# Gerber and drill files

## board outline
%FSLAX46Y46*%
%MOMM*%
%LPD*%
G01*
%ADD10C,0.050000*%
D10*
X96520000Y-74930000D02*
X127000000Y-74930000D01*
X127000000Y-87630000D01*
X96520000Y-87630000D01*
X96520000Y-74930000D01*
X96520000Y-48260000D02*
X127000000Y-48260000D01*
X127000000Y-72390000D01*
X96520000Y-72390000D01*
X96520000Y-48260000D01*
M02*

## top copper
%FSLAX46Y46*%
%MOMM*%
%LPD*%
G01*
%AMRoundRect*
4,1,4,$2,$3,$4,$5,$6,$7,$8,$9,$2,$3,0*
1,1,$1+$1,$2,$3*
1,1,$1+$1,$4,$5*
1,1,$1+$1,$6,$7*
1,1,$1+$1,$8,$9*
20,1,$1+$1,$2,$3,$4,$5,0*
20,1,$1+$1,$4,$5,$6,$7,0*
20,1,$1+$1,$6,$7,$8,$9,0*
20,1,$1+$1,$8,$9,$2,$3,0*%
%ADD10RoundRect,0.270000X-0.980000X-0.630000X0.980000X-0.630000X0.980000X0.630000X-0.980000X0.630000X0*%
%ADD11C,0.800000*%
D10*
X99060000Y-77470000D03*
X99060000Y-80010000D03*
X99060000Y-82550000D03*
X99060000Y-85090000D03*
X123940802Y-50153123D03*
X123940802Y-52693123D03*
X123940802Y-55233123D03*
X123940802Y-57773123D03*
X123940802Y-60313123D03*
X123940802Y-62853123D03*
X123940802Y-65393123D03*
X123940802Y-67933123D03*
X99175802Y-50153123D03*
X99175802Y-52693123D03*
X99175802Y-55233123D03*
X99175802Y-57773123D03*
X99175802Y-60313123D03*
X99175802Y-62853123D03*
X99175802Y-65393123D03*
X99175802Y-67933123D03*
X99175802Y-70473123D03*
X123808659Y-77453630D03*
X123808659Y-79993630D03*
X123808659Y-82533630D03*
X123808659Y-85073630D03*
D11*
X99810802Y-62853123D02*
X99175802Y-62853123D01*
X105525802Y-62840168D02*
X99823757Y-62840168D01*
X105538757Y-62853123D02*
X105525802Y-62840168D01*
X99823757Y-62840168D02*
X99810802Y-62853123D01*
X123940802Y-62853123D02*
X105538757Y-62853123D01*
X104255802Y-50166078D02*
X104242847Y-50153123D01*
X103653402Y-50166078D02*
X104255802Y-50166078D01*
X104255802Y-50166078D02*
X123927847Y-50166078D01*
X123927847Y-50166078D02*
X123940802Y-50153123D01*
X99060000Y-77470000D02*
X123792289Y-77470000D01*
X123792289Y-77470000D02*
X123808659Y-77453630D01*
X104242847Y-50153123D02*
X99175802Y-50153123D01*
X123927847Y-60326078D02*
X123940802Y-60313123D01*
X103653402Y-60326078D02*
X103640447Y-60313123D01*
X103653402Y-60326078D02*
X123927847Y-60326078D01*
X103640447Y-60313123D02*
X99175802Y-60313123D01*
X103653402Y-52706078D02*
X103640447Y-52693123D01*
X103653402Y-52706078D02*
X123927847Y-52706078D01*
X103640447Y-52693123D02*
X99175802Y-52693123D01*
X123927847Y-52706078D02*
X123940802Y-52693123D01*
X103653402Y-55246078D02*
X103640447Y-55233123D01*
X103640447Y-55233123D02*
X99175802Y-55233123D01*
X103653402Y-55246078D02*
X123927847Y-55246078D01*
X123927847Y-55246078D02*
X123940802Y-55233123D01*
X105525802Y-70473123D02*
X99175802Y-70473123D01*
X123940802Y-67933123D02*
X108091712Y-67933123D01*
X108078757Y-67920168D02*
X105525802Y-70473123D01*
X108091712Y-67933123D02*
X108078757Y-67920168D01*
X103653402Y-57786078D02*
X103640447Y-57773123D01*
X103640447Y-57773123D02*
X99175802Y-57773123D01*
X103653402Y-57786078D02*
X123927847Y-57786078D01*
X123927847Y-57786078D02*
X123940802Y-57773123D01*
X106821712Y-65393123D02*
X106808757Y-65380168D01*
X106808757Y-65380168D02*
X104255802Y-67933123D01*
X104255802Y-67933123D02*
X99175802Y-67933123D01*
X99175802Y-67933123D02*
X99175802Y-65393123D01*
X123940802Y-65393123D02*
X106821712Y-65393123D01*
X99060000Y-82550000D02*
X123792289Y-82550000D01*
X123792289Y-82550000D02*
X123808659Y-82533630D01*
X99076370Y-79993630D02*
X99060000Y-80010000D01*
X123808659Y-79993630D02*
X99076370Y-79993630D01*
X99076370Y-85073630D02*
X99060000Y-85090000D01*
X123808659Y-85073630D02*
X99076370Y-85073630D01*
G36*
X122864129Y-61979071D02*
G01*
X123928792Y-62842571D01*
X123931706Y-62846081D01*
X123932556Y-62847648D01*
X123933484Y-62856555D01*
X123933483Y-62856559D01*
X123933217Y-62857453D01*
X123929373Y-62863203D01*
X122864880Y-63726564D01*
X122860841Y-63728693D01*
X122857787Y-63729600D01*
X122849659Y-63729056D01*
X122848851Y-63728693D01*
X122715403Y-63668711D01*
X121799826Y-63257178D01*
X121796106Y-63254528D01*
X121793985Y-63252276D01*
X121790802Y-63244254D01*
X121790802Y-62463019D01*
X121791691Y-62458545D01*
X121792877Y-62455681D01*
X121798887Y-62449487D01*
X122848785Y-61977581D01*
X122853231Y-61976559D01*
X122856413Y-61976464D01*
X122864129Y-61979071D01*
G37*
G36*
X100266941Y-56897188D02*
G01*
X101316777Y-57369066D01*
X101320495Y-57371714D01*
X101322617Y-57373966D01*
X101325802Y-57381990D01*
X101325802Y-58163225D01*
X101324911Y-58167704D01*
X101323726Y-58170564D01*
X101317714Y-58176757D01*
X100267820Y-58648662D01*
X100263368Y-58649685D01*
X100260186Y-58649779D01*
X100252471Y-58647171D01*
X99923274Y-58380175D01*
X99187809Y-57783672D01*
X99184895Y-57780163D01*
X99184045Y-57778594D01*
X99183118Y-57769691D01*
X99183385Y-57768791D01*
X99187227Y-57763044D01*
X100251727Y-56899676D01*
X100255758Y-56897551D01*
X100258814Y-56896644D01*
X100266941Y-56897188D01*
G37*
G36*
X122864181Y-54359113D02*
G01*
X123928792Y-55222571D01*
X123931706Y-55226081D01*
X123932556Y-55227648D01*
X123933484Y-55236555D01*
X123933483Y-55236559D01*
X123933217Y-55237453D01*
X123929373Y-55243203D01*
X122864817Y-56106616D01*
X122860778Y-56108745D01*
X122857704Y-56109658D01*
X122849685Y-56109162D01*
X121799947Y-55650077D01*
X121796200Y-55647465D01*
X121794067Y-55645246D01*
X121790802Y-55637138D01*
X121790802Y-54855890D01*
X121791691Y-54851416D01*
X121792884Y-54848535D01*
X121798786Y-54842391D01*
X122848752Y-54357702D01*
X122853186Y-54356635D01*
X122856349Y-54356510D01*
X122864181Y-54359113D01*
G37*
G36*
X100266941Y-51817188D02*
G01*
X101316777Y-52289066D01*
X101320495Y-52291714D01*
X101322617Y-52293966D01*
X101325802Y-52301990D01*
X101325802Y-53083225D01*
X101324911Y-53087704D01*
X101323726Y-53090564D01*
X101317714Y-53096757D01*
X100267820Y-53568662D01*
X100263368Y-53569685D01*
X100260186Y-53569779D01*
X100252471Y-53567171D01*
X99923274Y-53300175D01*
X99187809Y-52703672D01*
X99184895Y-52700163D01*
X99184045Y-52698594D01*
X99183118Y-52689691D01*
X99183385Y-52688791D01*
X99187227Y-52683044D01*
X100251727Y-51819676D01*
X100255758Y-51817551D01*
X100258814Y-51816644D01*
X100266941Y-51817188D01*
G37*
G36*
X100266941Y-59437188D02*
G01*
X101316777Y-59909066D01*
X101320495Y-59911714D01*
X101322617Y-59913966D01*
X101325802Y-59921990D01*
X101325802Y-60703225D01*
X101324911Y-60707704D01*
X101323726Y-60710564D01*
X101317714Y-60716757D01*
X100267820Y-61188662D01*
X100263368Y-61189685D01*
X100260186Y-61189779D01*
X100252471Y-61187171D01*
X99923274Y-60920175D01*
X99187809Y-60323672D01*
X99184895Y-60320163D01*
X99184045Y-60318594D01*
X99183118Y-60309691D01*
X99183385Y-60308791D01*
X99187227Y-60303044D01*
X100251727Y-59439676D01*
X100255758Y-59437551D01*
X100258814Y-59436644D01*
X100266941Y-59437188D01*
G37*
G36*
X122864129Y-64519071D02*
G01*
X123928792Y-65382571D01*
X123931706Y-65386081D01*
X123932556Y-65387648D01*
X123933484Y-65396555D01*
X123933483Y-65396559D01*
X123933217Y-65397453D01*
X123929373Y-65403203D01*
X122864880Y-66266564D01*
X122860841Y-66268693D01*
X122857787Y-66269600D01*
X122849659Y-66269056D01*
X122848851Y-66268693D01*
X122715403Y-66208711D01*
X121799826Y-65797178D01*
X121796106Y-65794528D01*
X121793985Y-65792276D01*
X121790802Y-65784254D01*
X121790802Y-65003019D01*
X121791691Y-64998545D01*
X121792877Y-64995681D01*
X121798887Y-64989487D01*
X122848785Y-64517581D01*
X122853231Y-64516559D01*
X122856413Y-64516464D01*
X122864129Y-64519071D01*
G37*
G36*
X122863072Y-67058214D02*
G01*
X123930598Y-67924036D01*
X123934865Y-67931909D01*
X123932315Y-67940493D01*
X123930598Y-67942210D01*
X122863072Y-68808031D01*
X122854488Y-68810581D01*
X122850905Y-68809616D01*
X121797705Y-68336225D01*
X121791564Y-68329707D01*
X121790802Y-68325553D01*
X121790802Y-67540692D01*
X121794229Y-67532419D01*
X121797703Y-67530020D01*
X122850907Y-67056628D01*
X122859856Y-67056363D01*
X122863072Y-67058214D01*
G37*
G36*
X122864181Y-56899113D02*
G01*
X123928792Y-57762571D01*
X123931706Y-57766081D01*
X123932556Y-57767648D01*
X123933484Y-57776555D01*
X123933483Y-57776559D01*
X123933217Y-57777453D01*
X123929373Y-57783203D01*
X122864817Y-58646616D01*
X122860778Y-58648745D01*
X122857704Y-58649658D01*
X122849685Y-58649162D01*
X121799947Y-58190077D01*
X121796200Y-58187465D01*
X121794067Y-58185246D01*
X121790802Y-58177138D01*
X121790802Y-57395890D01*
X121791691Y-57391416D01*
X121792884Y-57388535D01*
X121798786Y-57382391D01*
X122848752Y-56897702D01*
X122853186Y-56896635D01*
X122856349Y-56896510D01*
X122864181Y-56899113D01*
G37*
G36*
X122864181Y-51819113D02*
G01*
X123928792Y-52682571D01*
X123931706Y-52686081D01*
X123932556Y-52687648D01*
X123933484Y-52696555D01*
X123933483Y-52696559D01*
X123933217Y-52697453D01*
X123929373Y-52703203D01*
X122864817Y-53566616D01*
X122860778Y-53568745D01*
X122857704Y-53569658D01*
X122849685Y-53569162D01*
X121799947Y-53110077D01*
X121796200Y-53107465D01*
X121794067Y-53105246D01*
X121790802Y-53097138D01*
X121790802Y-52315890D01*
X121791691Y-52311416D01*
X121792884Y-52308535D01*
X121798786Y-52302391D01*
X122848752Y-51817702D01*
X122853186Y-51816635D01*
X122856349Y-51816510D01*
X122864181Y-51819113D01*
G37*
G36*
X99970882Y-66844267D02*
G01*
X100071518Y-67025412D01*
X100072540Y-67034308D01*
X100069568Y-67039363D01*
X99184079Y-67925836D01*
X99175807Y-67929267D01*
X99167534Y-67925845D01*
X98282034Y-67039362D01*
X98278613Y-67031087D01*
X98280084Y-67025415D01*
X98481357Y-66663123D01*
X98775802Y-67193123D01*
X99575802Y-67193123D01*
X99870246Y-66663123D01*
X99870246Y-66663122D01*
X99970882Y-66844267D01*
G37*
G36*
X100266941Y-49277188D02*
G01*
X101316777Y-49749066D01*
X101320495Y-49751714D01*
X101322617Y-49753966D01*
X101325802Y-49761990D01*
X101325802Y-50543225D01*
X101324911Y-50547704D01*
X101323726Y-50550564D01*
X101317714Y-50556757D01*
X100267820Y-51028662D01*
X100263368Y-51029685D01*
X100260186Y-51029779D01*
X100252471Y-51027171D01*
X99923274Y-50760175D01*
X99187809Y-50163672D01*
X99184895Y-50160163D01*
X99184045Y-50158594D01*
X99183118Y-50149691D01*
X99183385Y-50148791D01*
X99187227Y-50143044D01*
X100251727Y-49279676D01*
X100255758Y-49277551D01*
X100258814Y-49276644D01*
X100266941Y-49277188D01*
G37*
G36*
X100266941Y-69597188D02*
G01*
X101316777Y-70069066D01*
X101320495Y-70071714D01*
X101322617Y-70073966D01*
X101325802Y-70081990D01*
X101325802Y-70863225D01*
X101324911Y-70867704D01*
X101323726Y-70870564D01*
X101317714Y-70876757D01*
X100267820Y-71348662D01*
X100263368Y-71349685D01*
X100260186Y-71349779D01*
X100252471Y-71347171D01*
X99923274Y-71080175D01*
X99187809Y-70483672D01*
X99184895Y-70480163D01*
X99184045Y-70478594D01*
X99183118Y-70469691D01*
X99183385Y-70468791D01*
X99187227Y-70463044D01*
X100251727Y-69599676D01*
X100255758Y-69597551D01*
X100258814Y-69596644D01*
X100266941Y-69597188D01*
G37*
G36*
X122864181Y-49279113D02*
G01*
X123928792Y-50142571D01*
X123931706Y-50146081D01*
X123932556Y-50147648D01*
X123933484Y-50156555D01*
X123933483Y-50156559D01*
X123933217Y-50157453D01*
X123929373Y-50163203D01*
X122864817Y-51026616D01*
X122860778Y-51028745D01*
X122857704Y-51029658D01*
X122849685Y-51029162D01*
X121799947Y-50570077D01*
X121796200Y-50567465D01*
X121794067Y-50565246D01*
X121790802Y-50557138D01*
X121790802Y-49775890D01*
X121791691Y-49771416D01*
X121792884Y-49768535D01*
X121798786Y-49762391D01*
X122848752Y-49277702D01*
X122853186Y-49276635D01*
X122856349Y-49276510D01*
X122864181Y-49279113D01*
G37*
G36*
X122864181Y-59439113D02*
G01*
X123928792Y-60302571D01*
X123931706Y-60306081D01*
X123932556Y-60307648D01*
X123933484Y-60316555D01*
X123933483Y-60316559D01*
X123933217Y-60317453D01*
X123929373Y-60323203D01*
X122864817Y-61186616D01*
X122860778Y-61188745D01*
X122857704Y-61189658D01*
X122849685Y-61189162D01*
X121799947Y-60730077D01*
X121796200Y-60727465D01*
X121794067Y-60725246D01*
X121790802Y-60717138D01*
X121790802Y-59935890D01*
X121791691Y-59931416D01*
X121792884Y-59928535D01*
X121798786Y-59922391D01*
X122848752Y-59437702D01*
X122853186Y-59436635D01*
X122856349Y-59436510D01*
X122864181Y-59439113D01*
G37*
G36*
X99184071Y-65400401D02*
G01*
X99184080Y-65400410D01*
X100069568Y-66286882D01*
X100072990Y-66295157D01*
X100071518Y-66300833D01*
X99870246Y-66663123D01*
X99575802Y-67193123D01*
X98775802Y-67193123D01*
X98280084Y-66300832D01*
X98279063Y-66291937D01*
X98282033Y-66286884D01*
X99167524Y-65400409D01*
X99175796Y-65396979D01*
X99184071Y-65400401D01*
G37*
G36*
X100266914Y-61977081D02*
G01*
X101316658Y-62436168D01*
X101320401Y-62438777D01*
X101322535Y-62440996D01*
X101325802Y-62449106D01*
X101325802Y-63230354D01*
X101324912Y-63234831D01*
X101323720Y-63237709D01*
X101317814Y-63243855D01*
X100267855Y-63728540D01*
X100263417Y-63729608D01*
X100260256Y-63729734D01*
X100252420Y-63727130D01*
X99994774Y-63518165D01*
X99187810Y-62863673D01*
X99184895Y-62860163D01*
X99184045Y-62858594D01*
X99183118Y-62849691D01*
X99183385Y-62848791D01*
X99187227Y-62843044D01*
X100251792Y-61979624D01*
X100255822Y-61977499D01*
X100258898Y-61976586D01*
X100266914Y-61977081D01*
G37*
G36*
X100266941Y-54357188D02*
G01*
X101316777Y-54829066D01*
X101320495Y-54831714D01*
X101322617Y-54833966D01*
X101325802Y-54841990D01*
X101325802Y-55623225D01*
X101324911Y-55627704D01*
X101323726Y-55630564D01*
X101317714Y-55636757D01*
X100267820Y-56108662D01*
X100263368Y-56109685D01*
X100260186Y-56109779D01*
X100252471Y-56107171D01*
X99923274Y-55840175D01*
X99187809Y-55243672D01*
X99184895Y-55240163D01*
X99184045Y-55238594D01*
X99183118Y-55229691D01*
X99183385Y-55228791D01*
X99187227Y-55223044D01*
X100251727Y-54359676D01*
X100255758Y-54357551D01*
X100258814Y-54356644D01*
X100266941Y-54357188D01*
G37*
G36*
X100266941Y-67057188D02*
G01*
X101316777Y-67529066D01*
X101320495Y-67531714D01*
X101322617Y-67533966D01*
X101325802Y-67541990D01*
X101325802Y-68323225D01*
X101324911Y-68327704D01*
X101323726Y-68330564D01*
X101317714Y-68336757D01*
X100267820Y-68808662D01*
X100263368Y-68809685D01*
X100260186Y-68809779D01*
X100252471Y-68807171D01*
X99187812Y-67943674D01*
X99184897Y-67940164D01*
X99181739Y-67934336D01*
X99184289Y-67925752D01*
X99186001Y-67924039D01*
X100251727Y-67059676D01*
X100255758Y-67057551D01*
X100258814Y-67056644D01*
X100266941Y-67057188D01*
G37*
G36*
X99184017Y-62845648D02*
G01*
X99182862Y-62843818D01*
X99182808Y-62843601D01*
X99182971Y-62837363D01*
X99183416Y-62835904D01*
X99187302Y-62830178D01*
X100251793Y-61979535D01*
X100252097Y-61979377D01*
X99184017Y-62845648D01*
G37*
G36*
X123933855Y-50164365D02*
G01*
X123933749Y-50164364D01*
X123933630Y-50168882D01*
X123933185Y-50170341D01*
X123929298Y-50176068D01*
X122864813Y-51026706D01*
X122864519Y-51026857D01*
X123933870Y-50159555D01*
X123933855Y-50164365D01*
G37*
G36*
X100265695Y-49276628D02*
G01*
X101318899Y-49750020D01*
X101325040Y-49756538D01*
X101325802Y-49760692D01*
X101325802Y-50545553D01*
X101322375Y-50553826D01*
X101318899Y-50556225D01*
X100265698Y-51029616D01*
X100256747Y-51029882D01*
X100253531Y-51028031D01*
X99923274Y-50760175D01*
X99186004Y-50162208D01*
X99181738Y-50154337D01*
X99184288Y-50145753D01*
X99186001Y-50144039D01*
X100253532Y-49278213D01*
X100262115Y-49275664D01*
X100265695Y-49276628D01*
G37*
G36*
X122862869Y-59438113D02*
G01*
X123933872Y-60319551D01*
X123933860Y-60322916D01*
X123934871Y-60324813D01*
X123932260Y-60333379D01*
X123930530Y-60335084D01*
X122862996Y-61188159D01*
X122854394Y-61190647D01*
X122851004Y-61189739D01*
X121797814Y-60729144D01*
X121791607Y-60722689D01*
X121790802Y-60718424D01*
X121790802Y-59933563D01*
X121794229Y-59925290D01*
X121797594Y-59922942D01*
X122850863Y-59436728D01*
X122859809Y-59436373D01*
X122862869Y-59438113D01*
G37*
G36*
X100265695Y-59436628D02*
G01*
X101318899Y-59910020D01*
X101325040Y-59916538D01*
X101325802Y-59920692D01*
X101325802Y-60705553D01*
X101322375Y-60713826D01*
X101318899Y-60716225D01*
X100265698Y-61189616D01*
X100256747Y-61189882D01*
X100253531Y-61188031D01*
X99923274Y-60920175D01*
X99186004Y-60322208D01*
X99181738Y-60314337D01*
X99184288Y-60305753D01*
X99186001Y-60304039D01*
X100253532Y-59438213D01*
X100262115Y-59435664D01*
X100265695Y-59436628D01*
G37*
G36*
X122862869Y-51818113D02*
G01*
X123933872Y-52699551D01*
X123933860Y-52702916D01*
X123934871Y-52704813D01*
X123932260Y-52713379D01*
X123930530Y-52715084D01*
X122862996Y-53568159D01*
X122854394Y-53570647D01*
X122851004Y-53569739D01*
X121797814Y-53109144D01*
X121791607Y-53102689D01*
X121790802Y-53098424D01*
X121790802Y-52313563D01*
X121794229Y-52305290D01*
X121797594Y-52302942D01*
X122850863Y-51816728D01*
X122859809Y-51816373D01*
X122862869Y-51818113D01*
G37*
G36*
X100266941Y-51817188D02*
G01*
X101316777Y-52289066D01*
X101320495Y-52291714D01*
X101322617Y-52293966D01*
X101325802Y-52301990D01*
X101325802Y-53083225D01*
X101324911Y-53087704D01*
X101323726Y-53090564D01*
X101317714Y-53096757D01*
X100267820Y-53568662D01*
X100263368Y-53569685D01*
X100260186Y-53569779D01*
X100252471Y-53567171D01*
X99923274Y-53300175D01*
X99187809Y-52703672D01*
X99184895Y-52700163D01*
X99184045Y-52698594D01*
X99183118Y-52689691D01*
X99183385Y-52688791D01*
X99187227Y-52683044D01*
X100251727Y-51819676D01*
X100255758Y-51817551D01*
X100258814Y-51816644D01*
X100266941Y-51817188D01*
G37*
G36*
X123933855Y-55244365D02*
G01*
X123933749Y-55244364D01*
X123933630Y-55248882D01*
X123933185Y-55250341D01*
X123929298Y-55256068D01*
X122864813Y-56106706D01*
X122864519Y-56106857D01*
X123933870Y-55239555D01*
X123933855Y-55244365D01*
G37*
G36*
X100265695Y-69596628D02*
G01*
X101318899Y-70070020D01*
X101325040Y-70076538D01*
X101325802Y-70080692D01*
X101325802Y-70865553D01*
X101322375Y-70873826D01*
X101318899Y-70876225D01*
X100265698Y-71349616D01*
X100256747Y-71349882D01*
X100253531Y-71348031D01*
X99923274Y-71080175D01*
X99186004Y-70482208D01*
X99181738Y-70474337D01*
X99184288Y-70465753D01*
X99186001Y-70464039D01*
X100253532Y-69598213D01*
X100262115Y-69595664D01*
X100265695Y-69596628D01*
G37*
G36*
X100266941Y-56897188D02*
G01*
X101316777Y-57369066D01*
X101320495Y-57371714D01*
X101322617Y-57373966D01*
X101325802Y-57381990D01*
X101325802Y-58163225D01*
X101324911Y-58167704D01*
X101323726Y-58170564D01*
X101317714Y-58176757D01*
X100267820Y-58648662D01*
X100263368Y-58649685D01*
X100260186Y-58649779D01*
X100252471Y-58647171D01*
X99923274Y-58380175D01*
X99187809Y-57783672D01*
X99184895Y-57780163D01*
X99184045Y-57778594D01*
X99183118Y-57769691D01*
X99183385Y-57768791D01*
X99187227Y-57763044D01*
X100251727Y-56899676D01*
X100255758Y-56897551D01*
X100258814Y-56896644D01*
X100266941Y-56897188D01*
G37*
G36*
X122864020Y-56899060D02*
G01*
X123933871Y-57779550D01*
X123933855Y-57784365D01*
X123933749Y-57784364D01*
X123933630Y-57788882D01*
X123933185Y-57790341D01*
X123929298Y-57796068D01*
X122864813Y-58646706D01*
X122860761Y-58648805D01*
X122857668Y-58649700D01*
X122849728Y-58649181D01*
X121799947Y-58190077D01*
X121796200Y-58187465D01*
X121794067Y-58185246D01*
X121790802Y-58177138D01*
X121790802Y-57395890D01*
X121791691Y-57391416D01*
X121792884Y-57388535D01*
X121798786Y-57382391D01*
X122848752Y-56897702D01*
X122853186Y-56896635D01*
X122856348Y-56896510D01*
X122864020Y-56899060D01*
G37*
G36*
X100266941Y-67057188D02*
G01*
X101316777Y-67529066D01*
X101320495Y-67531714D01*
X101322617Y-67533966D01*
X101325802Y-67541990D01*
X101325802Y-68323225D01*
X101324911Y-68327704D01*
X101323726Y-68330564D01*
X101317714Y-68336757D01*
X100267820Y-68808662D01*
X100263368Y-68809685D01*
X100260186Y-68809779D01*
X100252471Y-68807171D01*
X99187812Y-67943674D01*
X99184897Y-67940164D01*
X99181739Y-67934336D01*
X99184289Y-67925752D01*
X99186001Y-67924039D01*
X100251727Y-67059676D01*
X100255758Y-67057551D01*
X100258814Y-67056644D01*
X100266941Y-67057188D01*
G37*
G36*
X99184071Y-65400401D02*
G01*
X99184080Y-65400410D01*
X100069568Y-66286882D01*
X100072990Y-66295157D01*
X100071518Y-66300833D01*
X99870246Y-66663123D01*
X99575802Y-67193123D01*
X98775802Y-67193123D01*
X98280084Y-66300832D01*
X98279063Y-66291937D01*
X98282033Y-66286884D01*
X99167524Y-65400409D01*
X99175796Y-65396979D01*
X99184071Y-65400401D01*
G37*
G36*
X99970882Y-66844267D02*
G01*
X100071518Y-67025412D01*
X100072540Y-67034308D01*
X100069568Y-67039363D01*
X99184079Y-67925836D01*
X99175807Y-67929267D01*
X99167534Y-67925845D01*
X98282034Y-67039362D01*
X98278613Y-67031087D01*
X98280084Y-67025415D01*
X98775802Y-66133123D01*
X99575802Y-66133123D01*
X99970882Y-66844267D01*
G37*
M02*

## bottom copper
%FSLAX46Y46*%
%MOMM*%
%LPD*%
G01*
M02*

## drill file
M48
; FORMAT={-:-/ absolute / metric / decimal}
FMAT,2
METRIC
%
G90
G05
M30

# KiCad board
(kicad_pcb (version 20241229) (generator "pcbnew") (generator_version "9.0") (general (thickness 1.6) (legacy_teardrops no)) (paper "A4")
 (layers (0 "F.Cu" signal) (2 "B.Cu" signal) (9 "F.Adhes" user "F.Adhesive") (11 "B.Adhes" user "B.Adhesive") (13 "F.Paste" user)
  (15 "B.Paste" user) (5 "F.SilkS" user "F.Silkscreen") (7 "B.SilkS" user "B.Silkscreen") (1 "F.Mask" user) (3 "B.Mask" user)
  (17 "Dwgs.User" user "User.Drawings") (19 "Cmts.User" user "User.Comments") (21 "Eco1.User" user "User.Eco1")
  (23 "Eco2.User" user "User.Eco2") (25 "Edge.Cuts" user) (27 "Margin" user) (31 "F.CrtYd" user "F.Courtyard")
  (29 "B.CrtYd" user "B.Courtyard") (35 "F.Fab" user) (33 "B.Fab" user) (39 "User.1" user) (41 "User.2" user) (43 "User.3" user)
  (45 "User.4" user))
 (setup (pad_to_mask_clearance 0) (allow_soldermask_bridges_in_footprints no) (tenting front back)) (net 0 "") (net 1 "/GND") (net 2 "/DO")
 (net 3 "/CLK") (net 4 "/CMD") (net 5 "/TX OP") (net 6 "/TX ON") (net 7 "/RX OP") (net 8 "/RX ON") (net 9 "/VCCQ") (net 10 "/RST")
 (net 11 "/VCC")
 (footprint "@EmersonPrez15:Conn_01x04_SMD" (layer "F.Cu") (at 99.06 77.47 -90)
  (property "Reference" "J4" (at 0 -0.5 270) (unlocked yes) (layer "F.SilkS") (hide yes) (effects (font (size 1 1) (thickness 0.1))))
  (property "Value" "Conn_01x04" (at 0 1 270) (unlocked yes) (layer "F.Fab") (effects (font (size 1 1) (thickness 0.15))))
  (pad "1" smd roundrect (at 0 0) (size 2.5 1.8) (layers "F.Cu" "F.Mask" "F.Paste") (roundrect_rratio 0.15) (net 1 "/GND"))
  (pad "2" smd roundrect (at 2.54 0) (size 2.5 1.8) (layers "F.Cu" "F.Mask" "F.Paste") (roundrect_rratio 0.15) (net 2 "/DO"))
  (pad "3" smd roundrect (at 5.08 0) (size 2.5 1.8) (layers "F.Cu" "F.Mask" "F.Paste") (roundrect_rratio 0.15) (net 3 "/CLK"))
  (pad "4" smd roundrect (at 7.62 0) (size 2.5 1.8) (layers "F.Cu" "F.Mask" "F.Paste") (roundrect_rratio 0.15) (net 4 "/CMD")))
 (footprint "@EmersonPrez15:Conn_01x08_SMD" (layer "F.Cu") (at 123.940802 50.153123 -90)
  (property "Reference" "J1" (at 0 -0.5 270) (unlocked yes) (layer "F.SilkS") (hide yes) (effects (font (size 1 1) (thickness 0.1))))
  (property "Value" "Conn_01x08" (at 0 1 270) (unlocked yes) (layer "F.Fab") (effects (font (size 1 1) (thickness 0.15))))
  (pad "1" smd roundrect (at 0 0) (size 2.5 1.8) (layers "F.Cu" "F.Mask" "F.Paste") (roundrect_rratio 0.15) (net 1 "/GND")
   (teardrops (best_length_ratio 0.5) (max_length 1) (best_width_ratio 1) (max_width 2) (curved_edges no) (filter_ratio 0.9) (enabled yes)
    (allow_two_segments yes) (prefer_zone_connections yes)))
  (pad "2" smd roundrect (at 2.54 0) (size 2.5 1.8) (layers "F.Cu" "F.Mask" "F.Paste") (roundrect_rratio 0.15) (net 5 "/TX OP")
   (teardrops (best_length_ratio 0.5) (max_length 1) (best_width_ratio 1) (max_width 2) (curved_edges no) (filter_ratio 0.9) (enabled yes)
    (allow_two_segments yes) (prefer_zone_connections yes)))
  (pad "3" smd roundrect (at 5.08 0) (size 2.5 1.8) (layers "F.Cu" "F.Mask" "F.Paste") (roundrect_rratio 0.15) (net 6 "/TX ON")
   (teardrops (best_length_ratio 0.5) (max_length 1) (best_width_ratio 1) (max_width 2) (curved_edges no) (filter_ratio 0.9) (enabled yes)
    (allow_two_segments yes) (prefer_zone_connections yes)))
  (pad "4" smd roundrect (at 7.62 0) (size 2.5 1.8) (layers "F.Cu" "F.Mask" "F.Paste") (roundrect_rratio 0.15) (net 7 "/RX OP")
   (teardrops (best_length_ratio 0.5) (max_length 1) (best_width_ratio 1) (max_width 2) (curved_edges no) (filter_ratio 0.9) (enabled yes)
    (allow_two_segments yes) (prefer_zone_connections yes)))
  (pad "5" smd roundrect (at 10.16 0) (size 2.5 1.8) (layers "F.Cu" "F.Mask" "F.Paste") (roundrect_rratio 0.15) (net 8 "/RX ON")
   (teardrops (best_length_ratio 0.5) (max_length 1) (best_width_ratio 1) (max_width 2) (curved_edges no) (filter_ratio 0.9) (enabled yes)
    (allow_two_segments yes) (prefer_zone_connections yes)))
  (pad "6" smd roundrect (at 12.7 0) (size 2.5 1.8) (layers "F.Cu" "F.Mask" "F.Paste") (roundrect_rratio 0.15) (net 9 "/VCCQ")
   (teardrops (best_length_ratio 0.5) (max_length 1) (best_width_ratio 1) (max_width 2) (curved_edges no) (filter_ratio 0.9) (enabled yes)
    (allow_two_segments yes) (prefer_zone_connections yes)))
  (pad "7" smd roundrect (at 15.24 0) (size 2.5 1.8) (layers "F.Cu" "F.Mask" "F.Paste") (roundrect_rratio 0.15) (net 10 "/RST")
   (teardrops (best_length_ratio 0.5) (max_length 1) (best_width_ratio 1) (max_width 2) (curved_edges no) (filter_ratio 0.9) (enabled yes)
    (allow_two_segments yes) (prefer_zone_connections yes)))
  (pad "8" smd roundrect (at 17.78 0) (size 2.5 1.8) (layers "F.Cu" "F.Mask" "F.Paste") (roundrect_rratio 0.15) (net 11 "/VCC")
   (teardrops (best_length_ratio 0.5) (max_length 1) (best_width_ratio 1) (max_width 2) (curved_edges no) (filter_ratio 0.9) (enabled yes)
    (allow_two_segments yes) (prefer_zone_connections yes))))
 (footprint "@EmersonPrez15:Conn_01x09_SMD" (layer "F.Cu") (at 99.175802 50.153123 -90)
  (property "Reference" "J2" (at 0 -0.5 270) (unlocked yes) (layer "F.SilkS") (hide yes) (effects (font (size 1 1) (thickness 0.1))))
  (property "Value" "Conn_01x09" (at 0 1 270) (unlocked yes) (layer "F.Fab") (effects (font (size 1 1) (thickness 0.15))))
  (pad "1" smd roundrect (at 0 0) (size 2.5 1.8) (layers "F.Cu" "F.Mask" "F.Paste") (roundrect_rratio 0.15) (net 1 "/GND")
   (teardrops (best_length_ratio 0.5) (max_length 1) (best_width_ratio 1) (max_width 2) (curved_edges no) (filter_ratio 0.9) (enabled yes)
    (allow_two_segments yes) (prefer_zone_connections yes)))
  (pad "2" smd roundrect (at 2.54 0) (size 2.5 1.8) (layers "F.Cu" "F.Mask" "F.Paste") (roundrect_rratio 0.15) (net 5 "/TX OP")
   (teardrops (best_length_ratio 0.5) (max_length 1) (best_width_ratio 1) (max_width 2) (curved_edges no) (filter_ratio 0.9) (enabled yes)
    (allow_two_segments yes) (prefer_zone_connections yes)))
  (pad "3" smd roundrect (at 5.08 0) (size 2.5 1.8) (layers "F.Cu" "F.Mask" "F.Paste") (roundrect_rratio 0.15) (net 6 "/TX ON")
   (teardrops (best_length_ratio 0.5) (max_length 1) (best_width_ratio 1) (max_width 2) (curved_edges no) (filter_ratio 0.9) (enabled yes)
    (allow_two_segments yes) (prefer_zone_connections yes)))
  (pad "4" smd roundrect (at 7.62 0) (size 2.5 1.8) (layers "F.Cu" "F.Mask" "F.Paste") (roundrect_rratio 0.15) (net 7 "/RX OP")
   (teardrops (best_length_ratio 0.5) (max_length 1) (best_width_ratio 1) (max_width 2) (curved_edges no) (filter_ratio 0.9) (enabled yes)
    (allow_two_segments yes) (prefer_zone_connections yes)))
  (pad "5" smd roundrect (at 10.16 0) (size 2.5 1.8) (layers "F.Cu" "F.Mask" "F.Paste") (roundrect_rratio 0.15) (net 8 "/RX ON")
   (teardrops (best_length_ratio 0.5) (max_length 1) (best_width_ratio 1) (max_width 2) (curved_edges no) (filter_ratio 0.9) (enabled yes)
    (allow_two_segments yes) (prefer_zone_connections yes)))
  (pad "6" smd roundrect (at 12.7 0) (size 2.5 1.8) (layers "F.Cu" "F.Mask" "F.Paste") (roundrect_rratio 0.15) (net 9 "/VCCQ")
   (teardrops (best_length_ratio 0.5) (max_length 1) (best_width_ratio 1) (max_width 2) (curved_edges no) (filter_ratio 0.9) (enabled yes)
    (allow_two_segments yes) (prefer_zone_connections yes)))
  (pad "7" smd roundrect (at 15.24 0) (size 2.5 1.8) (layers "F.Cu" "F.Mask" "F.Paste") (roundrect_rratio 0.15) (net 10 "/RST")
   (teardrops (best_length_ratio 0.5) (max_length 1) (best_width_ratio 1) (max_width 2) (curved_edges no) (filter_ratio 0.9) (enabled yes)
    (allow_two_segments yes) (prefer_zone_connections yes)))
  (pad "8" smd roundrect (at 17.78 0) (size 2.5 1.8) (layers "F.Cu" "F.Mask" "F.Paste") (roundrect_rratio 0.15) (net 10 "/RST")
   (teardrops (best_length_ratio 0.5) (max_length 1) (best_width_ratio 1) (max_width 2) (curved_edges no) (filter_ratio 0.9) (enabled yes)
    (allow_two_segments yes) (prefer_zone_connections yes)))
  (pad "9" smd roundrect (at 20.32 0) (size 2.5 1.8) (layers "F.Cu" "F.Mask" "F.Paste") (roundrect_rratio 0.15) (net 11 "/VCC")
   (teardrops (best_length_ratio 0.5) (max_length 1) (best_width_ratio 1) (max_width 2) (curved_edges no) (filter_ratio 0.9) (enabled yes)
    (allow_two_segments yes) (prefer_zone_connections yes))))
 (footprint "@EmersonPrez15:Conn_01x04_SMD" (layer "F.Cu") (at 123.808659 77.45363 -90)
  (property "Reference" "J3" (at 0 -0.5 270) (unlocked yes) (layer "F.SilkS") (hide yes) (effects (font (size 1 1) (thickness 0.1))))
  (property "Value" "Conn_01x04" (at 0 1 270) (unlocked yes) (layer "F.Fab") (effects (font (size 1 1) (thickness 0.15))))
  (pad "1" smd roundrect (at 0 0) (size 2.5 1.8) (layers "F.Cu" "F.Mask" "F.Paste") (roundrect_rratio 0.15) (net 1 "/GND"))
  (pad "2" smd roundrect (at 2.54 0) (size 2.5 1.8) (layers "F.Cu" "F.Mask" "F.Paste") (roundrect_rratio 0.15) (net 2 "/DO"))
  (pad "3" smd roundrect (at 5.08 0) (size 2.5 1.8) (layers "F.Cu" "F.Mask" "F.Paste") (roundrect_rratio 0.15) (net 3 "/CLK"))
  (pad "4" smd roundrect (at 7.62 0) (size 2.5 1.8) (layers "F.Cu" "F.Mask" "F.Paste") (roundrect_rratio 0.15) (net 4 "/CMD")))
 (gr_rect (start 96.52 74.93) (end 127 87.63) (stroke (width 0.05) (type default)) (fill no) (layer "Edge.Cuts"))
 (gr_rect (start 96.52 48.26) (end 127 72.39) (stroke (width 0.05) (type default)) (fill no) (layer "Edge.Cuts"))
 (segment (start 99.810802 62.853123) (end 99.175802 62.853123) (width 0.8) (layer "F.Cu") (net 9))
 (segment (start 105.525802 62.840168) (end 99.823757 62.840168) (width 0.8) (layer "F.Cu") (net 9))
 (segment (start 105.538757 62.853123) (end 105.525802 62.840168) (width 0.8) (layer "F.Cu") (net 9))
 (segment (start 99.823757 62.840168) (end 99.810802 62.853123) (width 0.8) (layer "F.Cu") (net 9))
 (segment (start 123.940802 62.853123) (end 105.538757 62.853123) (width 0.8) (layer "F.Cu") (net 9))
 (segment (start 104.255802 50.166078) (end 104.242847 50.153123) (width 0.8) (layer "F.Cu") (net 1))
 (segment (start 103.653402 50.166078) (end 104.255802 50.166078) (width 0.8) (layer "F.Cu") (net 1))
 (segment (start 104.255802 50.166078) (end 123.927847 50.166078) (width 0.8) (layer "F.Cu") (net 1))
 (segment (start 123.927847 50.166078) (end 123.940802 50.153123) (width 0.8) (layer "F.Cu") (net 1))
 (segment (start 99.06 77.47) (end 123.792289 77.47) (width 0.8) (layer "F.Cu") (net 1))
 (segment (start 123.792289 77.47) (end 123.808659 77.45363) (width 0.8) (layer "F.Cu") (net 1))
 (segment (start 104.242847 50.153123) (end 99.175802 50.153123) (width 0.8) (layer "F.Cu") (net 1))
 (segment (start 123.927847 60.326078) (end 123.940802 60.313123) (width 0.8) (layer "F.Cu") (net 8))
 (segment (start 103.653402 60.326078) (end 103.640447 60.313123) (width 0.8) (layer "F.Cu") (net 8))
 (segment (start 103.653402 60.326078) (end 123.927847 60.326078) (width 0.8) (layer "F.Cu") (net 8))
 (segment (start 103.640447 60.313123) (end 99.175802 60.313123) (width 0.8) (layer "F.Cu") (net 8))
 (segment (start 103.653402 52.706078) (end 103.640447 52.693123) (width 0.8) (layer "F.Cu") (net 5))
 (segment (start 103.653402 52.706078) (end 123.927847 52.706078) (width 0.8) (layer "F.Cu") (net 5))
 (segment (start 103.640447 52.693123) (end 99.175802 52.693123) (width 0.8) (layer "F.Cu") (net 5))
 (segment (start 123.927847 52.706078) (end 123.940802 52.693123) (width 0.8) (layer "F.Cu") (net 5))
 (segment (start 103.653402 55.246078) (end 103.640447 55.233123) (width 0.8) (layer "F.Cu") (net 6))
 (segment (start 103.640447 55.233123) (end 99.175802 55.233123) (width 0.8) (layer "F.Cu") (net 6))
 (segment (start 103.653402 55.246078) (end 123.927847 55.246078) (width 0.8) (layer "F.Cu") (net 6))
 (segment (start 123.927847 55.246078) (end 123.940802 55.233123) (width 0.8) (layer "F.Cu") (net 6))
 (segment (start 105.525802 70.473123) (end 99.175802 70.473123) (width 0.8) (layer "F.Cu") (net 11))
 (segment (start 123.940802 67.933123) (end 108.091712 67.933123) (width 0.8) (layer "F.Cu") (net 11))
 (segment (start 108.078757 67.920168) (end 105.525802 70.473123) (width 0.8) (layer "F.Cu") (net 11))
 (segment (start 108.091712 67.933123) (end 108.078757 67.920168) (width 0.8) (layer "F.Cu") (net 11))
 (segment (start 103.653402 57.786078) (end 103.640447 57.773123) (width 0.8) (layer "F.Cu") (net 7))
 (segment (start 103.640447 57.773123) (end 99.175802 57.773123) (width 0.8) (layer "F.Cu") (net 7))
 (segment (start 103.653402 57.786078) (end 123.927847 57.786078) (width 0.8) (layer "F.Cu") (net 7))
 (segment (start 123.927847 57.786078) (end 123.940802 57.773123) (width 0.8) (layer "F.Cu") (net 7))
 (segment (start 106.821712 65.393123) (end 106.808757 65.380168) (width 0.8) (layer "F.Cu") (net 10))
 (segment (start 106.808757 65.380168) (end 104.255802 67.933123) (width 0.8) (layer "F.Cu") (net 10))
 (segment (start 104.255802 67.933123) (end 99.175802 67.933123) (width 0.8) (layer "F.Cu") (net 10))
 (segment (start 99.175802 67.933123) (end 99.175802 65.393123) (width 0.8) (layer "F.Cu") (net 10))
 (segment (start 123.940802 65.393123) (end 106.821712 65.393123) (width 0.8) (layer "F.Cu") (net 10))
 (segment (start 99.06 82.55) (end 123.792289 82.55) (width 0.8) (layer "F.Cu") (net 3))
 (segment (start 123.792289 82.55) (end 123.808659 82.53363) (width 0.8) (layer "F.Cu") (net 3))
 (segment (start 99.07637 79.99363) (end 99.06 80.01) (width 0.8) (layer "F.Cu") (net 2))
 (segment (start 123.808659 79.99363) (end 99.07637 79.99363) (width 0.8) (layer "F.Cu") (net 2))
 (segment (start 99.07637 85.07363) (end 99.06 85.09) (width 0.8) (layer "F.Cu") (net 4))
 (segment (start 123.808659 85.07363) (end 99.07637 85.07363) (width 0.8) (layer "F.Cu") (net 4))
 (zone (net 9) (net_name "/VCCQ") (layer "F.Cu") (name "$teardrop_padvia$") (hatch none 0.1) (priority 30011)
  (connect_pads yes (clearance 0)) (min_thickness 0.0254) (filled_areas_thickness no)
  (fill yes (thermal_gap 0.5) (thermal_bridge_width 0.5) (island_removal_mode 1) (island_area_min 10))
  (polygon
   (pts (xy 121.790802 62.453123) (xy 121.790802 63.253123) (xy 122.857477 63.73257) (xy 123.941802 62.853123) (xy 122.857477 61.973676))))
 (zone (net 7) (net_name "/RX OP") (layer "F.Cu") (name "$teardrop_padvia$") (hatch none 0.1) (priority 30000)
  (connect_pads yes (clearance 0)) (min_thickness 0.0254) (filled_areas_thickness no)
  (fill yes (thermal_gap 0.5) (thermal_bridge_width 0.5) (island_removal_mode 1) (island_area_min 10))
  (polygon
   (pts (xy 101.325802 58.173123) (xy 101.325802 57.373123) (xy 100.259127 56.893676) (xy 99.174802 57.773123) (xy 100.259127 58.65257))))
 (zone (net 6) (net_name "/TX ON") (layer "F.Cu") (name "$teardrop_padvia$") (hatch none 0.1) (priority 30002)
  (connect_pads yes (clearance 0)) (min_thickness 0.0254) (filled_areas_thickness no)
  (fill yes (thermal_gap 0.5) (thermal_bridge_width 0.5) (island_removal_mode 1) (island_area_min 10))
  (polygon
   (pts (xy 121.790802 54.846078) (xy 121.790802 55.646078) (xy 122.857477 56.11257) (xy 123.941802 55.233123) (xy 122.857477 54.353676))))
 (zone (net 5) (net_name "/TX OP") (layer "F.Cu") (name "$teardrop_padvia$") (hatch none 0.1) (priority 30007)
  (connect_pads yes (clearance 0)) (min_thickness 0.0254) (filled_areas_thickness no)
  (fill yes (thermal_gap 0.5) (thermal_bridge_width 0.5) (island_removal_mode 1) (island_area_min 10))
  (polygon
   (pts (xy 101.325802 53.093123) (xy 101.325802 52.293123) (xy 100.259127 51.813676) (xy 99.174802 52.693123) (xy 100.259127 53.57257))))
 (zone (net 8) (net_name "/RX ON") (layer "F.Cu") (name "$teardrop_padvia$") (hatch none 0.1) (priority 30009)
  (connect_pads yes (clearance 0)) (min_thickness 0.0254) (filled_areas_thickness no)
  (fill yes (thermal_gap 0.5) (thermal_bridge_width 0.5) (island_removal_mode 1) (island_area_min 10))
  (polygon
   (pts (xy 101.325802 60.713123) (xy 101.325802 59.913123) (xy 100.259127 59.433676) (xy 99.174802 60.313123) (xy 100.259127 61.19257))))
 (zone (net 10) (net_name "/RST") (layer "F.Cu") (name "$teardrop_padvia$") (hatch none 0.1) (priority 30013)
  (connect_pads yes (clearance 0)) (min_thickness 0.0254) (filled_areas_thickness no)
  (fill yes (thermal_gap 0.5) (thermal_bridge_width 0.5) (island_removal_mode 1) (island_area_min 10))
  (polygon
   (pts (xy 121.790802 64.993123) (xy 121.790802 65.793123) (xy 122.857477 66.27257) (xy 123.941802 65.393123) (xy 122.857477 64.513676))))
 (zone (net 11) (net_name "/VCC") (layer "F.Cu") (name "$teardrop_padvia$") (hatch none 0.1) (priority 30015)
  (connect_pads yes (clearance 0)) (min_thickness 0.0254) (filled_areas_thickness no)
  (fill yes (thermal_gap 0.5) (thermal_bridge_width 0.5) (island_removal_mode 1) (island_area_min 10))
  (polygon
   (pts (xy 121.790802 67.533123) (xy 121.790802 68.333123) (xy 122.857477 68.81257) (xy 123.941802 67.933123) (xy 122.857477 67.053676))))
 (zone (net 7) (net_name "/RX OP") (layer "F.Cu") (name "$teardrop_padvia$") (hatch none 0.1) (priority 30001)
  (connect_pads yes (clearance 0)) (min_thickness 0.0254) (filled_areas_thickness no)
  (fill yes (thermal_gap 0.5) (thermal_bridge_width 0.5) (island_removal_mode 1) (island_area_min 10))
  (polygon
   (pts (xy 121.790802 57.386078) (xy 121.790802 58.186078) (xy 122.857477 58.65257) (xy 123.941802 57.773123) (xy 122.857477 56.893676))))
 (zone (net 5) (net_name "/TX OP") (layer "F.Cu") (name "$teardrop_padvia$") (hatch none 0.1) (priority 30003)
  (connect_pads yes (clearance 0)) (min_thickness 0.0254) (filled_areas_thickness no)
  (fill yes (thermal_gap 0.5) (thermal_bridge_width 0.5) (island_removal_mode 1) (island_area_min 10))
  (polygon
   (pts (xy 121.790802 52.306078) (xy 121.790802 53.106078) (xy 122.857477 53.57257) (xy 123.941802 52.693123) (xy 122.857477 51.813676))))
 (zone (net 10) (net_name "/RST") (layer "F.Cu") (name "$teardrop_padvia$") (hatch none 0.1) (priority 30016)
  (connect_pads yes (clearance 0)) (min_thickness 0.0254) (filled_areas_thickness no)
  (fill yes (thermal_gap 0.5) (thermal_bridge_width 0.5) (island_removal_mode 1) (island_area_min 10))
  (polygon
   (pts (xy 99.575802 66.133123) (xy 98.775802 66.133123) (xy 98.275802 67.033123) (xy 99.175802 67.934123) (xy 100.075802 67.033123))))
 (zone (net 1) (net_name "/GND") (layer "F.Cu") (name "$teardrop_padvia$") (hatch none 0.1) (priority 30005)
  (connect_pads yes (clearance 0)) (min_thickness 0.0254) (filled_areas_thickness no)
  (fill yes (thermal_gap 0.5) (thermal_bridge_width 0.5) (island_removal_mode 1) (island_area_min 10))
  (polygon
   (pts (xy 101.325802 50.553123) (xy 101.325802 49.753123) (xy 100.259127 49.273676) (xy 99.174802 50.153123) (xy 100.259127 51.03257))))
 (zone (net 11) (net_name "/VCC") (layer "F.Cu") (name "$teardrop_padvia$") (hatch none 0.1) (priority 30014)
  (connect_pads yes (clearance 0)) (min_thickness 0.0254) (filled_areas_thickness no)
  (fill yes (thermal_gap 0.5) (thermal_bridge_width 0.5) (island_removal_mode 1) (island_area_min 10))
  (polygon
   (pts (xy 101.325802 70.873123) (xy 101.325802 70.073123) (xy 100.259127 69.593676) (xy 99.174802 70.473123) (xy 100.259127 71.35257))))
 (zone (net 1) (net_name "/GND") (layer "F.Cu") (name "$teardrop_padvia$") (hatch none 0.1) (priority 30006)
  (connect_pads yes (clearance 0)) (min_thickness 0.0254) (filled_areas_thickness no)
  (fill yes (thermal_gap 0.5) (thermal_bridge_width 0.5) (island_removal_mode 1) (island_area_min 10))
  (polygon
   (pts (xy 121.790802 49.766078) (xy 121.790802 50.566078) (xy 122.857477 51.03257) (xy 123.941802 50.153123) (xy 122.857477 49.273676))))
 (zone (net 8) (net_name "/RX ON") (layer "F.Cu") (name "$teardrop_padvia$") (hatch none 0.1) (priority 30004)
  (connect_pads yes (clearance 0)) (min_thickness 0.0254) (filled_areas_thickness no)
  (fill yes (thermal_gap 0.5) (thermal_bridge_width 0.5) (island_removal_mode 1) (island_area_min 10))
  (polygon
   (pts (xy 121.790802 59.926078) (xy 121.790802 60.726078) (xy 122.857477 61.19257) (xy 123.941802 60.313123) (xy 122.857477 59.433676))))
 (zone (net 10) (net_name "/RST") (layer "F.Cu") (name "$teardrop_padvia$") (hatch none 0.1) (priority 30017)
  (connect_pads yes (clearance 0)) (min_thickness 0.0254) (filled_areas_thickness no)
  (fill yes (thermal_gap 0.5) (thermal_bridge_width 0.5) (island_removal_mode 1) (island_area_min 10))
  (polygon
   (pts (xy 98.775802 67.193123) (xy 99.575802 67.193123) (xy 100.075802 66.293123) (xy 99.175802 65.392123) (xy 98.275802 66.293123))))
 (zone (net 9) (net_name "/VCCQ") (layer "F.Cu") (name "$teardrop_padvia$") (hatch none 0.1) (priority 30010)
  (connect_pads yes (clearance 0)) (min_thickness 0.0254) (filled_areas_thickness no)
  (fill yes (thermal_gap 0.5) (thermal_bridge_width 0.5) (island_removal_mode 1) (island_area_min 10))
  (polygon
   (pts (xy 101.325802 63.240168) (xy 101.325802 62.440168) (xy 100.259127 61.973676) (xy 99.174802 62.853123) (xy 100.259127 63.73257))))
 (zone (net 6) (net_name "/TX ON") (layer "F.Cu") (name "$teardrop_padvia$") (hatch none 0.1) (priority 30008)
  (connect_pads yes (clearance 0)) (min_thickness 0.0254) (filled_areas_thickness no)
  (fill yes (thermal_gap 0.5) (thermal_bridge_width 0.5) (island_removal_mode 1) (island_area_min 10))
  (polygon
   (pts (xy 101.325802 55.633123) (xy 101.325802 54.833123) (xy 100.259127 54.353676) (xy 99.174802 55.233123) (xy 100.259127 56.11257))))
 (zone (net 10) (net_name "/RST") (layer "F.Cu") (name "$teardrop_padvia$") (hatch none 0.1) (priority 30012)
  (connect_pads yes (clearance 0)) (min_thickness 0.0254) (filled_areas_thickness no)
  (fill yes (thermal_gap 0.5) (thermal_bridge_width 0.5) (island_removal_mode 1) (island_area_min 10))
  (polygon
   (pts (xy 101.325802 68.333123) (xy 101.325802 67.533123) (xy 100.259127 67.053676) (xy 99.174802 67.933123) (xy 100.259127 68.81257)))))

